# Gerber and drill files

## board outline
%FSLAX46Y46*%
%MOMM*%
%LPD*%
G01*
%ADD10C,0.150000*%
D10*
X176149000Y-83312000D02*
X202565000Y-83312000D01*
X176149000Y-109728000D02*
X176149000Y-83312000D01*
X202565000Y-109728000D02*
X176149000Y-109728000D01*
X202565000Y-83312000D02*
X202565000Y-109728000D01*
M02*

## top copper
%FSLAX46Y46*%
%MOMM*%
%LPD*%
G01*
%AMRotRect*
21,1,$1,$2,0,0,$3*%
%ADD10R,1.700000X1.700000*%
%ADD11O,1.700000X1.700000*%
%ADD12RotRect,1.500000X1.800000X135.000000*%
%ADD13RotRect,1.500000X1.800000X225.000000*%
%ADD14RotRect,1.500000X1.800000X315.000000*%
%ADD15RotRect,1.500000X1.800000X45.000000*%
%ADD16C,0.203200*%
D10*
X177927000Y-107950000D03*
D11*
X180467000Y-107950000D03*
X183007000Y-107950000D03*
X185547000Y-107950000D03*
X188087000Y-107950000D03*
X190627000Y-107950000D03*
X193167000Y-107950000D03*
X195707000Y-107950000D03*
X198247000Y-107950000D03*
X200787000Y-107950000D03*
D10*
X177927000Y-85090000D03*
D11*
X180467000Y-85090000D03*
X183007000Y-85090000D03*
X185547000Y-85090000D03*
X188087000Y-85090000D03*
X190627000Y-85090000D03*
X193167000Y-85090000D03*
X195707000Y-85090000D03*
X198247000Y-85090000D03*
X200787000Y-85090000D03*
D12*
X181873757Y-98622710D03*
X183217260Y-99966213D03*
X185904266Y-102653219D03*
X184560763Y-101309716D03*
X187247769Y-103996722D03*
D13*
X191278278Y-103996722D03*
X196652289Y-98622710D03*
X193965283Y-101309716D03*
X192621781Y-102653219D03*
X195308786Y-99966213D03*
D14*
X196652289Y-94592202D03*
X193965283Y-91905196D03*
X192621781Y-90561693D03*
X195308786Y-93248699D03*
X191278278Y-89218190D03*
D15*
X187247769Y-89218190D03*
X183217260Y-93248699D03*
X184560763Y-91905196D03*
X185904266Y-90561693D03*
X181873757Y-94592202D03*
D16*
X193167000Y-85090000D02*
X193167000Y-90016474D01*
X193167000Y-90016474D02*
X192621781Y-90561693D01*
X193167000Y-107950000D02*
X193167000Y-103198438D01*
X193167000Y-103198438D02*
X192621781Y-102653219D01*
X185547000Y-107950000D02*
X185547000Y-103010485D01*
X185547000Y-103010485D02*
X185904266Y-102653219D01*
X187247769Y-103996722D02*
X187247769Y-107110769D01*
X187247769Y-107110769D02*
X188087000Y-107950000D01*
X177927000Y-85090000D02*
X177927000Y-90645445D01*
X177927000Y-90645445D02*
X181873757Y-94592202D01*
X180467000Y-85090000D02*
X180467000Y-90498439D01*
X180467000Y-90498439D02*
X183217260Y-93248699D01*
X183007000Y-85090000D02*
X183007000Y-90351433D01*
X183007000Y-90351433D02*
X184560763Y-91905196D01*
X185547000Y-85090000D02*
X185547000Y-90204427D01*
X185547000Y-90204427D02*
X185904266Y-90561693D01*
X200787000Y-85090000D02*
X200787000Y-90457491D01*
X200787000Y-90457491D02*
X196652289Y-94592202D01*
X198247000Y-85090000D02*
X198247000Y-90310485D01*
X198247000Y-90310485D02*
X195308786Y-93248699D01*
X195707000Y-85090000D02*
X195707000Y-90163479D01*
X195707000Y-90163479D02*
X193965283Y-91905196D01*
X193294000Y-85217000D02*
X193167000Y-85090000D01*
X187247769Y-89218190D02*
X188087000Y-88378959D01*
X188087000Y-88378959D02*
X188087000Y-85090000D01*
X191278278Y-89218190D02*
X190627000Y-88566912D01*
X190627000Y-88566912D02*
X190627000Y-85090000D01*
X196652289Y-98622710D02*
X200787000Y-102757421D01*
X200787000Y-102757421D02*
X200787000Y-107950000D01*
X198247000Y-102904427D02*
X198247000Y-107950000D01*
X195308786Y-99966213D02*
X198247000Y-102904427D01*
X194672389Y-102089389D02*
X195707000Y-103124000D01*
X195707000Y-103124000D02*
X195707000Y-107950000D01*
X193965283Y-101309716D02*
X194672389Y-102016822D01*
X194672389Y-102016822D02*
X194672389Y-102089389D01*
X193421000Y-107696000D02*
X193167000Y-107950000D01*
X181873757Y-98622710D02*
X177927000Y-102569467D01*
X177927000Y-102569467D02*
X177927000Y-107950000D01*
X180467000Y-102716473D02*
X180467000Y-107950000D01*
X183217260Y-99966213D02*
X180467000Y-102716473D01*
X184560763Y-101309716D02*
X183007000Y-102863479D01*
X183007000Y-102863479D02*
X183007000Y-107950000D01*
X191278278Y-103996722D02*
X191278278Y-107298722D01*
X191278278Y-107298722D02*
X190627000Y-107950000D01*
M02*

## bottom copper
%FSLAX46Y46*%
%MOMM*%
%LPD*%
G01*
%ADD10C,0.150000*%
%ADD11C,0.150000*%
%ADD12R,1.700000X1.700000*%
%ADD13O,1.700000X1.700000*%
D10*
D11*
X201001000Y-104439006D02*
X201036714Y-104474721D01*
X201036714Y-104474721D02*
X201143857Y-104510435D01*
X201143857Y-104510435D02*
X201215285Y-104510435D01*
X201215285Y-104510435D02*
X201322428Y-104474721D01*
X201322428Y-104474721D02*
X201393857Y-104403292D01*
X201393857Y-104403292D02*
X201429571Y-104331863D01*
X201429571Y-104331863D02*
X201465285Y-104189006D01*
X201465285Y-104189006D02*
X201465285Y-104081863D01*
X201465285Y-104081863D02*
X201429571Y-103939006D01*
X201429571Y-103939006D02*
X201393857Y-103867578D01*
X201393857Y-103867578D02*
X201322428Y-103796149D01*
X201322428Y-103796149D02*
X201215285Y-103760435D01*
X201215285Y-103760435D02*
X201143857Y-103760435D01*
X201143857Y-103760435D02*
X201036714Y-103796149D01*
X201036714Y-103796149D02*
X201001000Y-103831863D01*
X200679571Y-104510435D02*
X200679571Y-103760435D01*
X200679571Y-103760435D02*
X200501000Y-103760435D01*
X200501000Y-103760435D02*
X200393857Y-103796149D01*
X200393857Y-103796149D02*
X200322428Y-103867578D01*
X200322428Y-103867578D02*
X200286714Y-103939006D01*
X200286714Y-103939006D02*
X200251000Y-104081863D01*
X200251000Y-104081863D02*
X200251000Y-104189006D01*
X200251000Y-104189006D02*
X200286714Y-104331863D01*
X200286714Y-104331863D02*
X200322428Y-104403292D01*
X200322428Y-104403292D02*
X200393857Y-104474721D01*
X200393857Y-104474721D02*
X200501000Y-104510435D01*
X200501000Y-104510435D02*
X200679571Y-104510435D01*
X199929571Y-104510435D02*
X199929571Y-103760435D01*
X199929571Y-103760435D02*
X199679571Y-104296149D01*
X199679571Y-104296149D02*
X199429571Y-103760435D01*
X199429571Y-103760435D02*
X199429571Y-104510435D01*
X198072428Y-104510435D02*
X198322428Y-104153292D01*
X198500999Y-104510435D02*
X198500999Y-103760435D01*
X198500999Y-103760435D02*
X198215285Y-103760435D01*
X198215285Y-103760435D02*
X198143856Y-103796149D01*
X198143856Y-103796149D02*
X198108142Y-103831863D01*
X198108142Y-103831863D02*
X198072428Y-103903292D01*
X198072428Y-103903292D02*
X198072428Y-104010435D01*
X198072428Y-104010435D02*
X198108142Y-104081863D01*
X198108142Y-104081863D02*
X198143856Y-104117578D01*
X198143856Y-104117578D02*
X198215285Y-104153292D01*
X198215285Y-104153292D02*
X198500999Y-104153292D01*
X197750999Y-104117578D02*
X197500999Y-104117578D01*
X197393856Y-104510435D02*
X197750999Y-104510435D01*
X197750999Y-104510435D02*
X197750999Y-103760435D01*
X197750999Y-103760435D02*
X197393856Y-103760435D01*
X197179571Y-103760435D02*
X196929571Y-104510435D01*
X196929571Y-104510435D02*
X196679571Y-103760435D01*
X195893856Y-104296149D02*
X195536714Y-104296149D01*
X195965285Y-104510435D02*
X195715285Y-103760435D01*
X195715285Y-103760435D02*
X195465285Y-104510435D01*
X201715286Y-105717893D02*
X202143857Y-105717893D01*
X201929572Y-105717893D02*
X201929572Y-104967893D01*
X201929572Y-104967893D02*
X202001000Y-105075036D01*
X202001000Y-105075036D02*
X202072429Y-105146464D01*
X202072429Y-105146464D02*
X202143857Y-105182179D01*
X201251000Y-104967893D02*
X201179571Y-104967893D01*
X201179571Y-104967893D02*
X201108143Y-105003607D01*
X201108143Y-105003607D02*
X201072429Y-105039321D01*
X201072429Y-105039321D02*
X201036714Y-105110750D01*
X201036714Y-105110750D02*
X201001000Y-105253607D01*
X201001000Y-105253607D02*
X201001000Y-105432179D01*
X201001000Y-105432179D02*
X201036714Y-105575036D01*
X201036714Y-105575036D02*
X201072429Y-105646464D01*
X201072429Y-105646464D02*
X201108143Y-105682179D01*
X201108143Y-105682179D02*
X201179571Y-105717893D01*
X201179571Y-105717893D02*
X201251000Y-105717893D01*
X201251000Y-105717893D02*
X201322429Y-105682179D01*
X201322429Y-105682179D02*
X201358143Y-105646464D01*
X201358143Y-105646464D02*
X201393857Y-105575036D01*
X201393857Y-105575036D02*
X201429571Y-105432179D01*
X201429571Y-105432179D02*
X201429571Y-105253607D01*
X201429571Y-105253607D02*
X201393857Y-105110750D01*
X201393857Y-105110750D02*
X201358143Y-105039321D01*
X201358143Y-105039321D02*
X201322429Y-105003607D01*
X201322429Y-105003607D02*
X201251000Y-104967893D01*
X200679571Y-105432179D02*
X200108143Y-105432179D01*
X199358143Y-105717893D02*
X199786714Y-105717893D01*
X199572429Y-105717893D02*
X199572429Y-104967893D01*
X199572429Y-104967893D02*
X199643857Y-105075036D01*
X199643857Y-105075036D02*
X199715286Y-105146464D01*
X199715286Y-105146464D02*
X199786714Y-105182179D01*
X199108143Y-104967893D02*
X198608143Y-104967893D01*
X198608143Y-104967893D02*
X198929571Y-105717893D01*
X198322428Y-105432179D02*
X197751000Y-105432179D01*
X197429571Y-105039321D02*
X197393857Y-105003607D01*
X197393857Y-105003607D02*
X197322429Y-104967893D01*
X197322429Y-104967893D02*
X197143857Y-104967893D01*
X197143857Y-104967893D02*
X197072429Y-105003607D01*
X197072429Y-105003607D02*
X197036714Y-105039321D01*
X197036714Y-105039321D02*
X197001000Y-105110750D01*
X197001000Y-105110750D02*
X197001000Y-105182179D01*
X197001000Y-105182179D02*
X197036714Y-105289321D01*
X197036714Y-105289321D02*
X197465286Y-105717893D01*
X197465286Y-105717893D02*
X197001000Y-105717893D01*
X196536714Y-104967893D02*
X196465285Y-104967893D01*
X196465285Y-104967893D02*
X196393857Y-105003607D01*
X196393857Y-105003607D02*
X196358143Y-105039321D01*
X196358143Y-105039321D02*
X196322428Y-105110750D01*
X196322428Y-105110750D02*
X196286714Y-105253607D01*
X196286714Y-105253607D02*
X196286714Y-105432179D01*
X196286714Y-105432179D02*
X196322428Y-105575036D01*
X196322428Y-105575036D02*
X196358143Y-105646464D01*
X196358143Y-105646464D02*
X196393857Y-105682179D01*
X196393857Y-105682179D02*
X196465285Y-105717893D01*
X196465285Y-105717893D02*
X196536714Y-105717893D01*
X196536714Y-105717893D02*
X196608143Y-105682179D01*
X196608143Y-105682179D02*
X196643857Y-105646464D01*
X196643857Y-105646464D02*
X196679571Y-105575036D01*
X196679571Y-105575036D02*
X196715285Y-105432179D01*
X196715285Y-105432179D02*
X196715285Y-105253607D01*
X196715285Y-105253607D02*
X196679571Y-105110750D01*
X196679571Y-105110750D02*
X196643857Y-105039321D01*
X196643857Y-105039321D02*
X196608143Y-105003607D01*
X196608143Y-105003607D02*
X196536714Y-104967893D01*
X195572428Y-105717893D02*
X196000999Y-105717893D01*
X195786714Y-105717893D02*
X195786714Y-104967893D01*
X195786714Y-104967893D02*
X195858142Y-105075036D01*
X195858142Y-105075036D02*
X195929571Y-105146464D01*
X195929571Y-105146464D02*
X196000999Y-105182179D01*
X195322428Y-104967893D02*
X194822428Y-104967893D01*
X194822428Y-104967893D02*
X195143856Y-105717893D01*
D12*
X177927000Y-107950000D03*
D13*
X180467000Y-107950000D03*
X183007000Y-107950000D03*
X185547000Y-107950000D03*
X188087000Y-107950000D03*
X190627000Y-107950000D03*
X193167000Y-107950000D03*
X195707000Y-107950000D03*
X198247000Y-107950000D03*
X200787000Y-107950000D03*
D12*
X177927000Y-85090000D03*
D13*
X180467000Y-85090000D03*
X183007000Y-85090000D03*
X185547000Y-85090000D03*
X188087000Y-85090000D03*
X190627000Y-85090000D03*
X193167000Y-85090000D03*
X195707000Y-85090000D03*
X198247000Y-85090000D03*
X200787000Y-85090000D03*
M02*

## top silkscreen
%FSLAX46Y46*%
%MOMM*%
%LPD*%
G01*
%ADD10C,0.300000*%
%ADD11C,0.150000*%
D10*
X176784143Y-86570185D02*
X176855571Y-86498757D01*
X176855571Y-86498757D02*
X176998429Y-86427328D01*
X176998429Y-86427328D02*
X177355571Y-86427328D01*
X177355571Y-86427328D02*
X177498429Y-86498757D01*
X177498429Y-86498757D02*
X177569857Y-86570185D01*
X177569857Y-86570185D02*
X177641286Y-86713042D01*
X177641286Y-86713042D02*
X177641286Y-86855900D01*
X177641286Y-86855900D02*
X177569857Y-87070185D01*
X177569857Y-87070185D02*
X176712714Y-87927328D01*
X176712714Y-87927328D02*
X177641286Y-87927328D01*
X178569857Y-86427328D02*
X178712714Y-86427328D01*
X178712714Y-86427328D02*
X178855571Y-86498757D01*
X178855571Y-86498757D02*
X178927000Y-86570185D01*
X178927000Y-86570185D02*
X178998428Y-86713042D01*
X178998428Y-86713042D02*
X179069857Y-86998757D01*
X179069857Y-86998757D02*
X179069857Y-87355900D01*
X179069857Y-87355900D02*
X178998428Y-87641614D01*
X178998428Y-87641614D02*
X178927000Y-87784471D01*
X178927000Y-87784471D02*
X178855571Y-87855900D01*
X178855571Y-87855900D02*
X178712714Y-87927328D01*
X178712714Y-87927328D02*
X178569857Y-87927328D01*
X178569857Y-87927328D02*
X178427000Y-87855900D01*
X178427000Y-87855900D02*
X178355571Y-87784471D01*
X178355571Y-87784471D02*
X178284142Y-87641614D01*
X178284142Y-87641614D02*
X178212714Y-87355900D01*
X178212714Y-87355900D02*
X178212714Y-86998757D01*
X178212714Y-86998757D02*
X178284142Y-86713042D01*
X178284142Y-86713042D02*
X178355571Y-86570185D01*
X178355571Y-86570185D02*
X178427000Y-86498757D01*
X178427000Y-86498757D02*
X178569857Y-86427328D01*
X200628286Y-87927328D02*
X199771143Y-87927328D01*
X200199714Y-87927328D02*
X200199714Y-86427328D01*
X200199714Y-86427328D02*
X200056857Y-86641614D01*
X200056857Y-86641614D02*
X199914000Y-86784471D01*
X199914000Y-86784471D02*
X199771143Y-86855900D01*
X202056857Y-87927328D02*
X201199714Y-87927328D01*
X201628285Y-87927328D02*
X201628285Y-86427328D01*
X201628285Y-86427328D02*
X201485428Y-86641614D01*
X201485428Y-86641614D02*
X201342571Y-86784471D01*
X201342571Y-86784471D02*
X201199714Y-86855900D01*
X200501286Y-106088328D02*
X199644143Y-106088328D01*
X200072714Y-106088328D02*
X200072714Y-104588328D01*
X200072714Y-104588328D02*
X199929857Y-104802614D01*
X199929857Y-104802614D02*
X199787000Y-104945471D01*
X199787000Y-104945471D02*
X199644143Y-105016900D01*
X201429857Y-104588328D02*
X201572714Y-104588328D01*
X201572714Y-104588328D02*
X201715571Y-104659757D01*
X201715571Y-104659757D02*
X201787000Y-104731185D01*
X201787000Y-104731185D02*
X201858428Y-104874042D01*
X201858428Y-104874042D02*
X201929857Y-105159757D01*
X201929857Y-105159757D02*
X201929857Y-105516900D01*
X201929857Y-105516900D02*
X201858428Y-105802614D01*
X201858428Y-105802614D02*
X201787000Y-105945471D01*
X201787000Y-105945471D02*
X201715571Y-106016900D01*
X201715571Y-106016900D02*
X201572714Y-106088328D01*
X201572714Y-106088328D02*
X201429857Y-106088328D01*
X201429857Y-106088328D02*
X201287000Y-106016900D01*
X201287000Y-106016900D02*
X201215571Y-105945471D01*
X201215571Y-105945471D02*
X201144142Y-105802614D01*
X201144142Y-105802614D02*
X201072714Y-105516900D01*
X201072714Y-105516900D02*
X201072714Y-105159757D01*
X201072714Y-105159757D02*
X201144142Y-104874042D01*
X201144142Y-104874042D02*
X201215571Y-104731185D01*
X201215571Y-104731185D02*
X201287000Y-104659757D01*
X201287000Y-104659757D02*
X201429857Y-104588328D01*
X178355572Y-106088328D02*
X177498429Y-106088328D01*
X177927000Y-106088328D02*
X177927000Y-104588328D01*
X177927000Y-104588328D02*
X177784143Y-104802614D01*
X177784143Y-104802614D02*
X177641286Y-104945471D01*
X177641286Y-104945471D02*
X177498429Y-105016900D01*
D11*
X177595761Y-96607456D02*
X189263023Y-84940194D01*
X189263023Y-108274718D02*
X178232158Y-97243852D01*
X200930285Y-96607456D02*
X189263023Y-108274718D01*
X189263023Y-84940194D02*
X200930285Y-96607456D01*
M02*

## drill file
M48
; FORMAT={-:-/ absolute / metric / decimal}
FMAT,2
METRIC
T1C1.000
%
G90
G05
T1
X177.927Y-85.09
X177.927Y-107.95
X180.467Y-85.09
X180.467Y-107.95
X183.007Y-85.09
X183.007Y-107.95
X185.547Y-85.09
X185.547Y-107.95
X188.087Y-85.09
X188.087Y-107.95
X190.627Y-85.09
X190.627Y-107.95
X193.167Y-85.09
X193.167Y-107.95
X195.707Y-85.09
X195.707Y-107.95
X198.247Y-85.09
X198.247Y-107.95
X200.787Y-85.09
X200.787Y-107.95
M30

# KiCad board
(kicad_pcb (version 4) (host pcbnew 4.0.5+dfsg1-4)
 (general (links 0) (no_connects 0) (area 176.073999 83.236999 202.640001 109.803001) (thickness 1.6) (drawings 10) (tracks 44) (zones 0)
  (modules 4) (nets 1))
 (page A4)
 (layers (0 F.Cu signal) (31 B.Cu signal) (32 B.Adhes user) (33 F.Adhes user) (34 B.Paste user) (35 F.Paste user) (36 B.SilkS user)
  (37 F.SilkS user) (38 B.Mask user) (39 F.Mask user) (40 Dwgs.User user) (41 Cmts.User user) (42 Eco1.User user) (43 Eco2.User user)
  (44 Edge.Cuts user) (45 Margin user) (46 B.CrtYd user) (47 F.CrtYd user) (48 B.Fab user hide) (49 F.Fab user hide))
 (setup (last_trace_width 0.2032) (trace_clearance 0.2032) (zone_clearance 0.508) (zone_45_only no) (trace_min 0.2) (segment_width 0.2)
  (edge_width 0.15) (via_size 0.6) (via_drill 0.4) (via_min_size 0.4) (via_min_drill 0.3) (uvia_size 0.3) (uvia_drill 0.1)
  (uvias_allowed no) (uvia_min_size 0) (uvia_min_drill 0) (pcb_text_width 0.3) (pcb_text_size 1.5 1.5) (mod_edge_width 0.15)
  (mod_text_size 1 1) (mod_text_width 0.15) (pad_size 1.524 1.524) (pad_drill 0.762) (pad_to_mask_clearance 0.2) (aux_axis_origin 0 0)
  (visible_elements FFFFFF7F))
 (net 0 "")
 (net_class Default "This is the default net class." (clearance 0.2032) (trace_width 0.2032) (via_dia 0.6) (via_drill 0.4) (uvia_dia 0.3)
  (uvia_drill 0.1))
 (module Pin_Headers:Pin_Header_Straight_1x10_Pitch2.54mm (layer B.Cu) (at 177.927 107.95 270)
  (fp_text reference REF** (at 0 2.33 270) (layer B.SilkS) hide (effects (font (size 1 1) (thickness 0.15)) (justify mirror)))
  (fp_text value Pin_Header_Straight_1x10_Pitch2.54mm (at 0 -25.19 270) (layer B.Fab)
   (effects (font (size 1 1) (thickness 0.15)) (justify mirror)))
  (pad 1 thru_hole rect (at 0 0 270) (size 1.7 1.7) (drill 1) (layers *.Cu *.Mask))
  (pad 2 thru_hole oval (at 0 -2.54 270) (size 1.7 1.7) (drill 1) (layers *.Cu *.Mask))
  (pad 3 thru_hole oval (at 0 -5.08 270) (size 1.7 1.7) (drill 1) (layers *.Cu *.Mask))
  (pad 4 thru_hole oval (at 0 -7.62 270) (size 1.7 1.7) (drill 1) (layers *.Cu *.Mask))
  (pad 5 thru_hole oval (at 0 -10.16 270) (size 1.7 1.7) (drill 1) (layers *.Cu *.Mask))
  (pad 6 thru_hole oval (at 0 -12.7 270) (size 1.7 1.7) (drill 1) (layers *.Cu *.Mask))
  (pad 7 thru_hole oval (at 0 -15.24 270) (size 1.7 1.7) (drill 1) (layers *.Cu *.Mask))
  (pad 8 thru_hole oval (at 0 -17.78 270) (size 1.7 1.7) (drill 1) (layers *.Cu *.Mask))
  (pad 9 thru_hole oval (at 0 -20.32 270) (size 1.7 1.7) (drill 1) (layers *.Cu *.Mask))
  (pad 10 thru_hole oval (at 0 -22.86 270) (size 1.7 1.7) (drill 1) (layers *.Cu *.Mask)))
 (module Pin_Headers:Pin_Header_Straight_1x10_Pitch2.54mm (layer B.Cu) (at 177.927 85.09 270)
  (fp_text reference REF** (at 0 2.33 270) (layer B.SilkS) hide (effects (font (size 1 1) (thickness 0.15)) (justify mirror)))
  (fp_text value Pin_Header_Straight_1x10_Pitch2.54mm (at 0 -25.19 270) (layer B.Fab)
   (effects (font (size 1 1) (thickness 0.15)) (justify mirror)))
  (pad 1 thru_hole rect (at 0 0 270) (size 1.7 1.7) (drill 1) (layers *.Cu *.Mask))
  (pad 2 thru_hole oval (at 0 -2.54 270) (size 1.7 1.7) (drill 1) (layers *.Cu *.Mask))
  (pad 3 thru_hole oval (at 0 -5.08 270) (size 1.7 1.7) (drill 1) (layers *.Cu *.Mask))
  (pad 4 thru_hole oval (at 0 -7.62 270) (size 1.7 1.7) (drill 1) (layers *.Cu *.Mask))
  (pad 5 thru_hole oval (at 0 -10.16 270) (size 1.7 1.7) (drill 1) (layers *.Cu *.Mask))
  (pad 6 thru_hole oval (at 0 -12.7 270) (size 1.7 1.7) (drill 1) (layers *.Cu *.Mask))
  (pad 7 thru_hole oval (at 0 -15.24 270) (size 1.7 1.7) (drill 1) (layers *.Cu *.Mask))
  (pad 8 thru_hole oval (at 0 -17.78 270) (size 1.7 1.7) (drill 1) (layers *.Cu *.Mask))
  (pad 9 thru_hole oval (at 0 -20.32 270) (size 1.7 1.7) (drill 1) (layers *.Cu *.Mask))
  (pad 10 thru_hole oval (at 0 -22.86 270) (size 1.7 1.7) (drill 1) (layers *.Cu *.Mask)))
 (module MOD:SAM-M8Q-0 (layer F.Cu) (at 189.333734 96.607456 45)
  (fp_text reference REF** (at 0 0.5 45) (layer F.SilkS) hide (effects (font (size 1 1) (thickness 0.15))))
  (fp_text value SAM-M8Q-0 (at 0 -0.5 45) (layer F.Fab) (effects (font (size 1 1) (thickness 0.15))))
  (fp_line (start -8.3 -8.3) (end 8.2 -8.3) (layer F.SilkS) (width 0.15))
  (fp_line (start -8.3 8.2) (end -8.3 -7.4) (layer F.SilkS) (width 0.15))
  (fp_line (start 8.2 8.2) (end -8.3 8.2) (layer F.SilkS) (width 0.15))
  (fp_line (start 8.2 -8.3) (end 8.2 8.2) (layer F.SilkS) (width 0.15))
  (pad 1 smd rect (at -6.7 -3.85 135) (size 1.5 1.8) (layers F.Cu F.Paste F.Mask))
  (pad 2 smd rect (at -6.7 -1.95 135) (size 1.5 1.8) (layers F.Cu F.Paste F.Mask))
  (pad 4 smd rect (at -6.7 1.85 135) (size 1.5 1.8) (layers F.Cu F.Paste F.Mask))
  (pad 3 smd rect (at -6.7 -0.05 135) (size 1.5 1.8) (layers F.Cu F.Paste F.Mask))
  (pad 5 smd rect (at -6.7 3.75 135) (size 1.5 1.8) (layers F.Cu F.Paste F.Mask))
  (pad 6 smd rect (at -3.85 6.6 225) (size 1.5 1.8) (layers F.Cu F.Paste F.Mask))
  (pad 10 smd rect (at 3.75 6.6 225) (size 1.5 1.8) (layers F.Cu F.Paste F.Mask))
  (pad 8 smd rect (at -0.05 6.6 225) (size 1.5 1.8) (layers F.Cu F.Paste F.Mask))
  (pad 7 smd rect (at -1.95 6.6 225) (size 1.5 1.8) (layers F.Cu F.Paste F.Mask))
  (pad 9 smd rect (at 1.85 6.6 225) (size 1.5 1.8) (layers F.Cu F.Paste F.Mask))
  (pad 11 smd rect (at 6.6 3.75 315) (size 1.5 1.8) (layers F.Cu F.Paste F.Mask))
  (pad 13 smd rect (at 6.6 -0.05 315) (size 1.5 1.8) (layers F.Cu F.Paste F.Mask))
  (pad 14 smd rect (at 6.6 -1.95 315) (size 1.5 1.8) (layers F.Cu F.Paste F.Mask))
  (pad 12 smd rect (at 6.6 1.85 315) (size 1.5 1.8) (layers F.Cu F.Paste F.Mask))
  (pad 15 smd rect (at 6.6 -3.85 315) (size 1.5 1.8) (layers F.Cu F.Paste F.Mask))
  (pad 16 smd rect (at 3.75 -6.7 45) (size 1.5 1.8) (layers F.Cu F.Paste F.Mask))
  (pad 19 smd rect (at -1.95 -6.7 45) (size 1.5 1.8) (layers F.Cu F.Paste F.Mask))
  (pad 18 smd rect (at -0.05 -6.7 45) (size 1.5 1.8) (layers F.Cu F.Paste F.Mask))
  (pad 17 smd rect (at 1.85 -6.7 45) (size 1.5 1.8) (layers F.Cu F.Paste F.Mask))
  (pad 20 smd rect (at -3.85 -6.7 45) (size 1.5 1.8) (layers F.Cu F.Paste F.Mask)))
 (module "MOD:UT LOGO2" (layer B.Cu) (at 189.23 93.345 180)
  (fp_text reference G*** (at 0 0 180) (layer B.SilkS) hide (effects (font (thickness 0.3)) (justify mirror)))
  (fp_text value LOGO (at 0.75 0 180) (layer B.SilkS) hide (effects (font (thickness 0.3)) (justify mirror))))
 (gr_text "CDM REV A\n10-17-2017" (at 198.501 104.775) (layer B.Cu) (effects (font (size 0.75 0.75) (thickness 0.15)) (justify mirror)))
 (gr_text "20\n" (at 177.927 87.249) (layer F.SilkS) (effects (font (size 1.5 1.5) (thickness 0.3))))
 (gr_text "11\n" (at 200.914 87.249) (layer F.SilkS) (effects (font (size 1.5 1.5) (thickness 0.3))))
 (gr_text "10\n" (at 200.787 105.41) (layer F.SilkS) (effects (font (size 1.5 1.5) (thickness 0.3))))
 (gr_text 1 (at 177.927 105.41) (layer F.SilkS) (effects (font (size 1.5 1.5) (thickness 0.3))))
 (gr_line (start 176.149 83.312) (end 202.565 83.312) (layer Edge.Cuts) (width 0.15))
 (gr_line (start 176.149 109.728) (end 176.149 83.312) (layer Edge.Cuts) (width 0.15))
 (gr_line (start 202.565 109.728) (end 176.149 109.728) (layer Edge.Cuts) (width 0.15))
 (gr_line (start 202.565 83.312) (end 202.565 109.728) (layer Edge.Cuts) (width 0.15))
 (segment (start 193.167 85.09) (end 193.167 90.016474) (width 0.2032) (layer F.Cu) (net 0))
 (segment (start 193.167 90.016474) (end 192.621781 90.561693) (width 0.2032) (layer F.Cu) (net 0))
 (segment (start 193.167 107.95) (end 193.167 103.198438) (width 0.2032) (layer F.Cu) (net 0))
 (segment (start 193.167 103.198438) (end 192.621781 102.653219) (width 0.2032) (layer F.Cu) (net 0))
 (segment (start 185.547 107.95) (end 185.547 103.010485) (width 0.2032) (layer F.Cu) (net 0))
 (segment (start 185.547 103.010485) (end 185.904266 102.653219) (width 0.2032) (layer F.Cu) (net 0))
 (segment (start 187.247769 103.996722) (end 187.247769 107.110769) (width 0.2032) (layer F.Cu) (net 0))
 (segment (start 187.247769 107.110769) (end 188.087 107.95) (width 0.2032) (layer F.Cu) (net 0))
 (segment (start 177.927 85.09) (end 177.927 90.645445) (width 0.2032) (layer F.Cu) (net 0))
 (segment (start 177.927 90.645445) (end 181.873757 94.592202) (width 0.2032) (layer F.Cu) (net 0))
 (segment (start 180.467 85.09) (end 180.467 90.498439) (width 0.2032) (layer F.Cu) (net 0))
 (segment (start 180.467 90.498439) (end 183.21726 93.248699) (width 0.2032) (layer F.Cu) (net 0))
 (segment (start 183.007 85.09) (end 183.007 90.351433) (width 0.2032) (layer F.Cu) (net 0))
 (segment (start 183.007 90.351433) (end 184.560763 91.905196) (width 0.2032) (layer F.Cu) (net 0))
 (segment (start 185.547 85.09) (end 185.547 90.204427) (width 0.2032) (layer F.Cu) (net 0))
 (segment (start 185.547 90.204427) (end 185.904266 90.561693) (width 0.2032) (layer F.Cu) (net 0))
 (segment (start 200.787 85.09) (end 200.787 90.457491) (width 0.2032) (layer F.Cu) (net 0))
 (segment (start 200.787 90.457491) (end 196.652289 94.592202) (width 0.2032) (layer F.Cu) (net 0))
 (segment (start 198.247 85.09) (end 198.247 90.310485) (width 0.2032) (layer F.Cu) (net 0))
 (segment (start 198.247 90.310485) (end 195.308786 93.248699) (width 0.2032) (layer F.Cu) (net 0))
 (segment (start 195.707 85.09) (end 195.707 90.163479) (width 0.2032) (layer F.Cu) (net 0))
 (segment (start 195.707 90.163479) (end 193.965283 91.905196) (width 0.2032) (layer F.Cu) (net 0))
 (segment (start 193.294 85.217) (end 193.167 85.09) (width 0.2032) (layer F.Cu) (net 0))
 (segment (start 187.247769 89.21819) (end 188.087 88.378959) (width 0.2032) (layer F.Cu) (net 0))
 (segment (start 188.087 88.378959) (end 188.087 85.09) (width 0.2032) (layer F.Cu) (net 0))
 (segment (start 191.278278 89.21819) (end 190.627 88.566912) (width 0.2032) (layer F.Cu) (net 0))
 (segment (start 190.627 88.566912) (end 190.627 85.09) (width 0.2032) (layer F.Cu) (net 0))
 (segment (start 196.652289 98.62271) (end 200.787 102.757421) (width 0.2032) (layer F.Cu) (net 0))
 (segment (start 200.787 102.757421) (end 200.787 107.95) (width 0.2032) (layer F.Cu) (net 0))
 (segment (start 198.247 102.904427) (end 198.247 107.95) (width 0.2032) (layer F.Cu) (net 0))
 (segment (start 195.308786 99.966213) (end 198.247 102.904427) (width 0.2032) (layer F.Cu) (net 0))
 (segment (start 194.672389 102.089389) (end 195.707 103.124) (width 0.2032) (layer F.Cu) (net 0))
 (segment (start 195.707 103.124) (end 195.707 107.95) (width 0.2032) (layer F.Cu) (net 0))
 (segment (start 193.965283 101.309716) (end 194.672389 102.016822) (width 0.2032) (layer F.Cu) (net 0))
 (segment (start 194.672389 102.016822) (end 194.672389 102.089389) (width 0.2032) (layer F.Cu) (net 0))
 (segment (start 193.421 107.696) (end 193.167 107.95) (width 0.2032) (layer F.Cu) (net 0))
 (segment (start 181.873757 98.62271) (end 177.927 102.569467) (width 0.2032) (layer F.Cu) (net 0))
 (segment (start 177.927 102.569467) (end 177.927 107.95) (width 0.2032) (layer F.Cu) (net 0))
 (segment (start 180.467 102.716473) (end 180.467 107.95) (width 0.2032) (layer F.Cu) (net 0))
 (segment (start 183.21726 99.966213) (end 180.467 102.716473) (width 0.2032) (layer F.Cu) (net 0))
 (segment (start 184.560763 101.309716) (end 183.007 102.863479) (width 0.2032) (layer F.Cu) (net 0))
 (segment (start 183.007 102.863479) (end 183.007 107.95) (width 0.2032) (layer F.Cu) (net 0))
 (segment (start 191.278278 103.996722) (end 191.278278 107.298722) (width 0.2032) (layer F.Cu) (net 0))
 (segment (start 191.278278 107.298722) (end 190.627 107.95) (width 0.2032) (layer F.Cu) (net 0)))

